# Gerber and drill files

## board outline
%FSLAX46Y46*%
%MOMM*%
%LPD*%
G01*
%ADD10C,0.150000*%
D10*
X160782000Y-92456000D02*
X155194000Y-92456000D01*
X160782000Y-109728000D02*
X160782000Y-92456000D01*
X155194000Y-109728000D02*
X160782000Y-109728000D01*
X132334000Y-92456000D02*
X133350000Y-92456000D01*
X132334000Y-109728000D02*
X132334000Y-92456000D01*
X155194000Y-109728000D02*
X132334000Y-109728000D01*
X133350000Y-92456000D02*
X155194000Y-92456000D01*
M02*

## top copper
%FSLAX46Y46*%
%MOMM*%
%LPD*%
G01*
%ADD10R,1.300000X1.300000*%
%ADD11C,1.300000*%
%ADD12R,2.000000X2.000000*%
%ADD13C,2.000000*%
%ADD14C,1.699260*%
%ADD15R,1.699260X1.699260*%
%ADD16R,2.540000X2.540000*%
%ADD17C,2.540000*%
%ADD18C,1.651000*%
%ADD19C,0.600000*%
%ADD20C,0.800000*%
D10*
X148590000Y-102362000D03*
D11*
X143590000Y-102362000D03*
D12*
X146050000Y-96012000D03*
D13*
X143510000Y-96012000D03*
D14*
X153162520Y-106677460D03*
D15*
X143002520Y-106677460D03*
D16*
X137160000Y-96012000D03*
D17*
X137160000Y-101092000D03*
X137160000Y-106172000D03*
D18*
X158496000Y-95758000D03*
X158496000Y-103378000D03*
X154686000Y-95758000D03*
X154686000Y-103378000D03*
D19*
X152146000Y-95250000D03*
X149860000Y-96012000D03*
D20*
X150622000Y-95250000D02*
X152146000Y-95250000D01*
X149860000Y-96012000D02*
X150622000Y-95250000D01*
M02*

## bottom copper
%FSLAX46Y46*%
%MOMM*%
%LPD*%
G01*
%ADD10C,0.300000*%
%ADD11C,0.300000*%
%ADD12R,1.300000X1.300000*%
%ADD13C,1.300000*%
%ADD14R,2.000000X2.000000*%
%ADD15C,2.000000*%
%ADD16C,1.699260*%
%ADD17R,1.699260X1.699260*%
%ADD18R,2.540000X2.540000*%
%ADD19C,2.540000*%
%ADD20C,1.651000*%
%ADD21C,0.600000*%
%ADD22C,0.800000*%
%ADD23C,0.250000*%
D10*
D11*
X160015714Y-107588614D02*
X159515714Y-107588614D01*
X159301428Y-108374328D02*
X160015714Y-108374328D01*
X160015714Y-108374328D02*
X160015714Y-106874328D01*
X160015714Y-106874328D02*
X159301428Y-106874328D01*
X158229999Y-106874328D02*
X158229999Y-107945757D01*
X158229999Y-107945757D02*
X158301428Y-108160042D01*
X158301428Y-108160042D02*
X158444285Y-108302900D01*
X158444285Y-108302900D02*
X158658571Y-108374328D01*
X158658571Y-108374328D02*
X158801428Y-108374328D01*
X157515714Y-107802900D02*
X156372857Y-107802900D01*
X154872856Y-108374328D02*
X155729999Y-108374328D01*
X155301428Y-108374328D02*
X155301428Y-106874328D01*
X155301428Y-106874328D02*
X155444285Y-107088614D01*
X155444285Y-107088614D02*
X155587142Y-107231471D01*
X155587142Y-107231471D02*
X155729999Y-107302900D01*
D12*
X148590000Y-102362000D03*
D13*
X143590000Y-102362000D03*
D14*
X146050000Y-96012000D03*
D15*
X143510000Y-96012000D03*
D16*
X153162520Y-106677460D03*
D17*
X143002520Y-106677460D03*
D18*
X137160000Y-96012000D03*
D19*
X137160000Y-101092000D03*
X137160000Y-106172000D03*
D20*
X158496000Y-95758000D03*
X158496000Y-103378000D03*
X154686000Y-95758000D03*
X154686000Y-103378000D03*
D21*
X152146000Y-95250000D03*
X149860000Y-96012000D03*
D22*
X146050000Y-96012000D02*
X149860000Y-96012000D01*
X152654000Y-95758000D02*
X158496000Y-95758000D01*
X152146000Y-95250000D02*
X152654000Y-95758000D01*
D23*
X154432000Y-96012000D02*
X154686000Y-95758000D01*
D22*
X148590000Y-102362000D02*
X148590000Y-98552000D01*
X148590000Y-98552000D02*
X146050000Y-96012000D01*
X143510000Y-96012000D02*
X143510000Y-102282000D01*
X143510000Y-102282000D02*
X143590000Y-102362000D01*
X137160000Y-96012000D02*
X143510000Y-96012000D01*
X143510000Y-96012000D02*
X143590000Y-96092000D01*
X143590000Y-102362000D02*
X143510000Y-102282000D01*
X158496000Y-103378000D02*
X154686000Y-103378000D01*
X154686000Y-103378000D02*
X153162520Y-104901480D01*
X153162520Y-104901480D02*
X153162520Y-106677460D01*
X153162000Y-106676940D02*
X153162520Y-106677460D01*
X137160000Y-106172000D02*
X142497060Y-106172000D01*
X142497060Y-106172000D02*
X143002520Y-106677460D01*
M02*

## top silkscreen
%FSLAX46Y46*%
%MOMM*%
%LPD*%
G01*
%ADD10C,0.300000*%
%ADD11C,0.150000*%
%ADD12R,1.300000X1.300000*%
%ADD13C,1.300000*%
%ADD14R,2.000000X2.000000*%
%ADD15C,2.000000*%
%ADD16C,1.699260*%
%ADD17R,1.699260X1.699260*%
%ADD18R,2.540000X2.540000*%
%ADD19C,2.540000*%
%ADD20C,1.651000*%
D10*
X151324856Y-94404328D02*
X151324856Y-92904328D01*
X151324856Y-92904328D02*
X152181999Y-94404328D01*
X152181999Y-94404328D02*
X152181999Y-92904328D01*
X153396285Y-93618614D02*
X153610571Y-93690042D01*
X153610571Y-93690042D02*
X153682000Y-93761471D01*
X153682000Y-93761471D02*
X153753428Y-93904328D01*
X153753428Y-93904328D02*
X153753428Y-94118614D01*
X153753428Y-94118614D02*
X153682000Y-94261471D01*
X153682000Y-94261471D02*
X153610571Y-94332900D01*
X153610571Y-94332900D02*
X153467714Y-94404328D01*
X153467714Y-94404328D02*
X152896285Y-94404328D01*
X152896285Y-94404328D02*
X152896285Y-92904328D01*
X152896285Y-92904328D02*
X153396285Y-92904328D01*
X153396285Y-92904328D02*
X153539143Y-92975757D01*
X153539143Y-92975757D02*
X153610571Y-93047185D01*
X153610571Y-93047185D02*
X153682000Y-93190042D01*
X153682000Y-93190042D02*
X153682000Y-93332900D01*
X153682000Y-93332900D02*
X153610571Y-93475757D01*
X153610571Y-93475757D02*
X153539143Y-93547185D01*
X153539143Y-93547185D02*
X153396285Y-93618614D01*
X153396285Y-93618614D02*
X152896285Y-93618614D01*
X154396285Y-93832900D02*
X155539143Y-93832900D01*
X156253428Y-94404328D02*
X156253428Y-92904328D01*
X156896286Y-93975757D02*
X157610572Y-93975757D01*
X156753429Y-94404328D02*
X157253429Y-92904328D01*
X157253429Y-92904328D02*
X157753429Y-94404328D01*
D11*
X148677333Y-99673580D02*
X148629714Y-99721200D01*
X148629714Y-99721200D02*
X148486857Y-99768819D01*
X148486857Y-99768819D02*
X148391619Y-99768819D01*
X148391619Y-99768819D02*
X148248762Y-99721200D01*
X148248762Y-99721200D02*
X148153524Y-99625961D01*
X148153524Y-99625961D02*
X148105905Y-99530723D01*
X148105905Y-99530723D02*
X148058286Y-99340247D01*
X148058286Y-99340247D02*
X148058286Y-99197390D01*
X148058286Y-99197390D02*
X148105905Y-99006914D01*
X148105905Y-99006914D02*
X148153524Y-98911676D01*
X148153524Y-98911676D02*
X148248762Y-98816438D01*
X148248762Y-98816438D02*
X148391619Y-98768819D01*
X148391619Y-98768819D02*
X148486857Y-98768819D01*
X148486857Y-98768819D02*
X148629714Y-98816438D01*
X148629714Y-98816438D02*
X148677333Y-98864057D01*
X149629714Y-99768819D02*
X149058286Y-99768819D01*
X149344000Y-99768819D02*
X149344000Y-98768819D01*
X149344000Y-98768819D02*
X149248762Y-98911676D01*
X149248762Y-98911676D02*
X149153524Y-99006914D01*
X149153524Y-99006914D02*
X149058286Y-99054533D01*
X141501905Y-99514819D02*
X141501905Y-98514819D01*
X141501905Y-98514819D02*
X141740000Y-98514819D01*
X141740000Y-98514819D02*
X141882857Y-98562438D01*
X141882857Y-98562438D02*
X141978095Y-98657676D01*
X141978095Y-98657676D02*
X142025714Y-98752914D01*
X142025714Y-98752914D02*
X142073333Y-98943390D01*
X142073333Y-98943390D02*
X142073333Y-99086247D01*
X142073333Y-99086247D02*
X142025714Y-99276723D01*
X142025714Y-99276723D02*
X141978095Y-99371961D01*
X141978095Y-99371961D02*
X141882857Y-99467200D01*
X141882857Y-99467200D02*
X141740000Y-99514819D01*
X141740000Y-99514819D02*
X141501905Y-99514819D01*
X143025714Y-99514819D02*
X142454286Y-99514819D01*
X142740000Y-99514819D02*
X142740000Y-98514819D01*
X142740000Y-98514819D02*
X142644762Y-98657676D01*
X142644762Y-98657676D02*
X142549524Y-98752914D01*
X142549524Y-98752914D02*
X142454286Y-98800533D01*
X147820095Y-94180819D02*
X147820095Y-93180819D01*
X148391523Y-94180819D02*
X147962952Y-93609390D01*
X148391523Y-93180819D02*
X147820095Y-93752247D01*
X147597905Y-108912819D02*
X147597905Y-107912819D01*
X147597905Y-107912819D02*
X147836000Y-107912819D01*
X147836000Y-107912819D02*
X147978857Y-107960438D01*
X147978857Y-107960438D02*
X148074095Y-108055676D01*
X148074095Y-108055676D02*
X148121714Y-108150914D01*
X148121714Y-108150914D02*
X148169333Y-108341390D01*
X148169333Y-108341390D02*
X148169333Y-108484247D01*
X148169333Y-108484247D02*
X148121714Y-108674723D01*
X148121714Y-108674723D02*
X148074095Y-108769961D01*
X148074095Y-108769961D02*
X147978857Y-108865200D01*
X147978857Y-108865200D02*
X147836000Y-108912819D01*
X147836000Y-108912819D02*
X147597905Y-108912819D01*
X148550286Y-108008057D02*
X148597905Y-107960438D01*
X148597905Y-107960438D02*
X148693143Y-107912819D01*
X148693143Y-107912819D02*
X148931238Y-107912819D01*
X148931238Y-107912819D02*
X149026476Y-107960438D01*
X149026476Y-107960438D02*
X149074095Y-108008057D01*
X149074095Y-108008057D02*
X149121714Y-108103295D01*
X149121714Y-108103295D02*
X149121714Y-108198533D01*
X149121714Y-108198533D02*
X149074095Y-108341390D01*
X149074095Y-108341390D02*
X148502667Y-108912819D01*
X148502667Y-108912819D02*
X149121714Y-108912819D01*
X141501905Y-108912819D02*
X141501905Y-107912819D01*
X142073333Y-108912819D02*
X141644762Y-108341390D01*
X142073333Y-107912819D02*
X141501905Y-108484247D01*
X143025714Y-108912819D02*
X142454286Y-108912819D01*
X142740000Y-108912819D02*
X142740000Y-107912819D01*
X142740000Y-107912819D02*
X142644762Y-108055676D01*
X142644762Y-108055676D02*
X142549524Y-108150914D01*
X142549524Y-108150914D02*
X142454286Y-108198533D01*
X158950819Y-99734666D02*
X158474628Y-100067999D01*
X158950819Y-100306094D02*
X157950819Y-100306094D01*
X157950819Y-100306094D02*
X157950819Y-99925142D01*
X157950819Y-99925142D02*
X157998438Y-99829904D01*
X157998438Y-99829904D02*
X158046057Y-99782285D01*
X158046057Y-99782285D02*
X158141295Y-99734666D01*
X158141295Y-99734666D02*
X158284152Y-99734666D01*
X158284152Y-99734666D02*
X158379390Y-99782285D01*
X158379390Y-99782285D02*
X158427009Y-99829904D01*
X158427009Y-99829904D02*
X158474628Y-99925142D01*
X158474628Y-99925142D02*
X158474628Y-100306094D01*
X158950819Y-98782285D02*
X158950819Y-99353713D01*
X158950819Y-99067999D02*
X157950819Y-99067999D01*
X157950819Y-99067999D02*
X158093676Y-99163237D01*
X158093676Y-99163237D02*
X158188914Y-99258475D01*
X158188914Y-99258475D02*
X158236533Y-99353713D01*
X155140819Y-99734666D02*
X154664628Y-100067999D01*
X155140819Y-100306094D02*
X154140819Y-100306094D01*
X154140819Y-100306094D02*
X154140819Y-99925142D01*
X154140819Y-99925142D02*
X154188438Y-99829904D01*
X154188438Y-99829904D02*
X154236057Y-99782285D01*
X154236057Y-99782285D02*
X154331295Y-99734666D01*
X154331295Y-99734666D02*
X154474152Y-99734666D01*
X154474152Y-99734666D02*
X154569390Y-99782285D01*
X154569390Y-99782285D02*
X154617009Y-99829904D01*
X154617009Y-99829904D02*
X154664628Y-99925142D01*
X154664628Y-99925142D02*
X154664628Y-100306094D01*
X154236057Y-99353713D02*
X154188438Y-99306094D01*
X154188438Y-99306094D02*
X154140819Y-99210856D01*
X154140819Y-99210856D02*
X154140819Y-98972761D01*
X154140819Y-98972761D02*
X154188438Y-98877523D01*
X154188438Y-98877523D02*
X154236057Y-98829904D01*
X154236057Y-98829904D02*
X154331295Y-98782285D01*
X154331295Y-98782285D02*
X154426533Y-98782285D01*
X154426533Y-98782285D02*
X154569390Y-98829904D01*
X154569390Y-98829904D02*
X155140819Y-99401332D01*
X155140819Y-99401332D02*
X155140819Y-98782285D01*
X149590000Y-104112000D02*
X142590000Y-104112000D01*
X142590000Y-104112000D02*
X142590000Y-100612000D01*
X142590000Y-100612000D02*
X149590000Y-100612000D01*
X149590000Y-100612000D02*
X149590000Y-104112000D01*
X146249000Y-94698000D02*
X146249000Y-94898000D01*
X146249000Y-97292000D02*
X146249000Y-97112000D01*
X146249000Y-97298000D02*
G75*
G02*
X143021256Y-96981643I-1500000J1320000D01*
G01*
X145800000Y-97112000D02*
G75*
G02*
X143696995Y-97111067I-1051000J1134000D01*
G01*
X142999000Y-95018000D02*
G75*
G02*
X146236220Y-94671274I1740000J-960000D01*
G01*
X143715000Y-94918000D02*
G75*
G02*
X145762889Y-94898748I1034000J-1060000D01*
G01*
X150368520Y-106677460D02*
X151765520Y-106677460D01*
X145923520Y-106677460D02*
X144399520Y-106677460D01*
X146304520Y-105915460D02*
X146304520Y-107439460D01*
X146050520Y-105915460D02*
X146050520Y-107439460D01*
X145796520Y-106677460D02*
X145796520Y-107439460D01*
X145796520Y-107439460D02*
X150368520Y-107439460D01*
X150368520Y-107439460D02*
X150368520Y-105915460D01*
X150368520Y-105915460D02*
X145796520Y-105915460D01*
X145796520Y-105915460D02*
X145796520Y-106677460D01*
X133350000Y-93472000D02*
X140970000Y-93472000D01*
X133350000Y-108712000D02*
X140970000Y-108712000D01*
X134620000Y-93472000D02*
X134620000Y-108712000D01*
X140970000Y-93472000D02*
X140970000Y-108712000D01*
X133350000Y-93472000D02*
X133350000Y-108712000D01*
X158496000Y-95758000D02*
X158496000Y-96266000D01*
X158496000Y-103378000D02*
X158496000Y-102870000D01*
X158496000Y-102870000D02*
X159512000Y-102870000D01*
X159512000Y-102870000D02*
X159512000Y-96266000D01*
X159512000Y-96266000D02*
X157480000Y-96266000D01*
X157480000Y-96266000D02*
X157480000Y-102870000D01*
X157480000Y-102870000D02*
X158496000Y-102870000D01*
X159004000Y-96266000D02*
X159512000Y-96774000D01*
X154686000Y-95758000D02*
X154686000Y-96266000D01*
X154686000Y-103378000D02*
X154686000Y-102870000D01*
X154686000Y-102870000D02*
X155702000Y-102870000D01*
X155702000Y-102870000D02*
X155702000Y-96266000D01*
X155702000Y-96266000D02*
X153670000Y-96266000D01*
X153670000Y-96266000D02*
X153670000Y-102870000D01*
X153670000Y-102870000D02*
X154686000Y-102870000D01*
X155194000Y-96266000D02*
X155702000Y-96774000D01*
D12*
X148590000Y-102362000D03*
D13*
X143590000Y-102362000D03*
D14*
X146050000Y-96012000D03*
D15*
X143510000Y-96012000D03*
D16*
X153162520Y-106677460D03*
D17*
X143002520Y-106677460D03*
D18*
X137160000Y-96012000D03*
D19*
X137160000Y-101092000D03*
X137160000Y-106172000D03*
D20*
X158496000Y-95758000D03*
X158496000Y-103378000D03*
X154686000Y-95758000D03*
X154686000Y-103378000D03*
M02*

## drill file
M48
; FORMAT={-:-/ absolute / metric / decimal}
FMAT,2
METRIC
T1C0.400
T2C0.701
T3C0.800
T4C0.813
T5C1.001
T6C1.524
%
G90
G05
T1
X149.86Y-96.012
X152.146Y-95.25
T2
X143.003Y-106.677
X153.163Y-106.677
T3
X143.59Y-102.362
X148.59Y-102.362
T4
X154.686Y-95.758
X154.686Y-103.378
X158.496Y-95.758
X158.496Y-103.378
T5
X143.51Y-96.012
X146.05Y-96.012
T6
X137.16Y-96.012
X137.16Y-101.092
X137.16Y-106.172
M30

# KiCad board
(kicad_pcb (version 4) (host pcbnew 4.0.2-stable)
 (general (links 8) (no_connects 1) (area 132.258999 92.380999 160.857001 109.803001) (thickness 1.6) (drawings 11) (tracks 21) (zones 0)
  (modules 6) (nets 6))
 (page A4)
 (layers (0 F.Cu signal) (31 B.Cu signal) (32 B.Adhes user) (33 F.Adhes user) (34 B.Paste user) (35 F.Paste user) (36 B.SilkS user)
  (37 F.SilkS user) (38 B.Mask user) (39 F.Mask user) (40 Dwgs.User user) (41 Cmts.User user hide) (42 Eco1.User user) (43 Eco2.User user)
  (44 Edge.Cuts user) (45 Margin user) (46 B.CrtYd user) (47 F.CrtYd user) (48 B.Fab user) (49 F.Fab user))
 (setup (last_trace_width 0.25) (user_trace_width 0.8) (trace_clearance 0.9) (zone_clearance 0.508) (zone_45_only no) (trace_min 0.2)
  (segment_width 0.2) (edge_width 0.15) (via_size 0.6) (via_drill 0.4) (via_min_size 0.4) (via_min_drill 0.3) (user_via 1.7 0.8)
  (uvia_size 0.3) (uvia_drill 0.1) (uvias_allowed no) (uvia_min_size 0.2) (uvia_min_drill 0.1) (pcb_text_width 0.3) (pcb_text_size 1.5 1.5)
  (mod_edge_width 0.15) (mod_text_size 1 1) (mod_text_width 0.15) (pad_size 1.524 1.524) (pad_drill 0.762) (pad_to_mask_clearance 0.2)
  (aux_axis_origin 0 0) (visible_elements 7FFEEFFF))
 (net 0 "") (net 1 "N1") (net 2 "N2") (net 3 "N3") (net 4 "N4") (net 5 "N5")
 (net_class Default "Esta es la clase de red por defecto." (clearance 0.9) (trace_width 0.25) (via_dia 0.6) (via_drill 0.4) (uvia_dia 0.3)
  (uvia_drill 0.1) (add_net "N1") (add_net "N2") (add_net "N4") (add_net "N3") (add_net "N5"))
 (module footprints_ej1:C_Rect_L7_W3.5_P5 (layer F.Cu) (at 148.59 102.362 180)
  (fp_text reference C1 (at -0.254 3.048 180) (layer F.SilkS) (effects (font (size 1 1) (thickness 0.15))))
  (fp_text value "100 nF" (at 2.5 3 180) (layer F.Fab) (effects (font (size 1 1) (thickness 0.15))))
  (fp_line (start -1 -1.75) (end 6 -1.75) (layer F.SilkS) (width 0.15))
  (fp_line (start 6 -1.75) (end 6 1.75) (layer F.SilkS) (width 0.15))
  (fp_line (start 6 1.75) (end -1 1.75) (layer F.SilkS) (width 0.15))
  (fp_line (start -1 1.75) (end -1 -1.75) (layer F.SilkS) (width 0.15))
  (pad 1 thru_hole rect (at 0 0 180) (size 1.3 1.3) (drill 0.8) (layers *.Cu *.Mask F.SilkS) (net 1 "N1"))
  (pad 2 thru_hole circle (at 5 0 180) (size 1.3 1.3) (drill 0.8) (layers *.Cu *.Mask F.SilkS) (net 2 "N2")))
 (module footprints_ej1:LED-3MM (layer F.Cu) (at 146.05 96.012 180)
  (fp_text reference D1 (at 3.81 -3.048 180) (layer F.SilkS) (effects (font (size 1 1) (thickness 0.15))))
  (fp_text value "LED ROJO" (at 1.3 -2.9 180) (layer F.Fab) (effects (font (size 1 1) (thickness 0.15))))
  (fp_line (start -0.199 1.314) (end -0.199 1.114) (layer F.SilkS) (width 0.15))
  (fp_line (start -0.199 -1.28) (end -0.199 -1.1) (layer F.SilkS) (width 0.15))
  (fp_arc (start 1.301 0.034) (end -0.199 -1.286) (angle 108.5) (layer F.SilkS) (width 0.15))
  (fp_arc (start 1.301 0.034) (end 0.25 -1.1) (angle 85.7) (layer F.SilkS) (width 0.15))
  (fp_arc (start 1.311 0.034) (end 3.051 0.994) (angle 110) (layer F.SilkS) (width 0.15))
  (fp_arc (start 1.301 0.034) (end 2.335 1.094) (angle 87.5) (layer F.SilkS) (width 0.15))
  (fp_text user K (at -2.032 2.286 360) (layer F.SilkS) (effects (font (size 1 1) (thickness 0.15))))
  (pad 1 thru_hole rect (at 0 0 270) (size 2 2) (drill 1.00076) (layers *.Cu *.Mask F.SilkS) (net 1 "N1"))
  (pad 2 thru_hole circle (at 2.54 0 180) (size 2 2) (drill 1.00076) (layers *.Cu *.Mask F.SilkS) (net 2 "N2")))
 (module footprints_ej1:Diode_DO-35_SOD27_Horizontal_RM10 (layer F.Cu) (at 143.002 106.68)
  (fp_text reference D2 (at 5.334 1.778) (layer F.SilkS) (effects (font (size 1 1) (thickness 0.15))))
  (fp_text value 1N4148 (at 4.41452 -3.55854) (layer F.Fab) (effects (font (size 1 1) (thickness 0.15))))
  (fp_line (start 7.36652 -0.00254) (end 8.76352 -0.00254) (layer F.SilkS) (width 0.15))
  (fp_line (start 2.92152 -0.00254) (end 1.39752 -0.00254) (layer F.SilkS) (width 0.15))
  (fp_line (start 3.30252 -0.76454) (end 3.30252 0.75946) (layer F.SilkS) (width 0.15))
  (fp_line (start 3.04852 -0.76454) (end 3.04852 0.75946) (layer F.SilkS) (width 0.15))
  (fp_line (start 2.79452 -0.00254) (end 2.79452 0.75946) (layer F.SilkS) (width 0.15))
  (fp_line (start 2.79452 0.75946) (end 7.36652 0.75946) (layer F.SilkS) (width 0.15))
  (fp_line (start 7.36652 0.75946) (end 7.36652 -0.76454) (layer F.SilkS) (width 0.15))
  (fp_line (start 7.36652 -0.76454) (end 2.79452 -0.76454) (layer F.SilkS) (width 0.15))
  (fp_line (start 2.79452 -0.76454) (end 2.79452 -0.00254) (layer F.SilkS) (width 0.15))
  (pad 2 thru_hole circle (at 10.16052 -0.00254 180) (size 1.69926 1.69926) (drill 0.70104) (layers *.Cu *.Mask F.SilkS) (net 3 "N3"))
  (pad 1 thru_hole rect (at 0.00052 -0.00254 180) (size 1.69926 1.69926) (drill 0.70104) (layers *.Cu *.Mask F.SilkS) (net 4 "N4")))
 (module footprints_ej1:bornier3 (layer F.Cu) (at 137.16 101.092 270)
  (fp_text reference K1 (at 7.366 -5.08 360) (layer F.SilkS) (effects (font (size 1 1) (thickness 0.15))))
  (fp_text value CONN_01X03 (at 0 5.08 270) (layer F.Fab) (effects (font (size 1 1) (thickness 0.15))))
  (fp_line (start -7.62 3.81) (end -7.62 -3.81) (layer F.SilkS) (width 0.15))
  (fp_line (start 7.62 3.81) (end 7.62 -3.81) (layer F.SilkS) (width 0.15))
  (fp_line (start -7.62 2.54) (end 7.62 2.54) (layer F.SilkS) (width 0.15))
  (fp_line (start -7.62 -3.81) (end 7.62 -3.81) (layer F.SilkS) (width 0.15))
  (fp_line (start -7.62 3.81) (end 7.62 3.81) (layer F.SilkS) (width 0.15))
  (pad 1 thru_hole rect (at -5.08 0 270) (size 2.54 2.54) (drill 1.524) (layers *.Cu *.Mask F.SilkS) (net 2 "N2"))
  (pad 2 thru_hole circle (at 0 0 270) (size 2.54 2.54) (drill 1.524) (layers *.Cu *.Mask F.SilkS) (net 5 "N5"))
  (pad 3 thru_hole circle (at 5.08 0 270) (size 2.54 2.54) (drill 1.524) (layers *.Cu *.Mask F.SilkS) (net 4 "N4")))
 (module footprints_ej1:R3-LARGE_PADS (layer F.Cu) (at 158.496 99.568 270)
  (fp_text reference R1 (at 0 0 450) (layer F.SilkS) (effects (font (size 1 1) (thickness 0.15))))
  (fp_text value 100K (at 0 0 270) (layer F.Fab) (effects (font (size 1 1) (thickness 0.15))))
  (fp_line (start -3.81 0) (end -3.302 0) (layer F.SilkS) (width 0.15))
  (fp_line (start 3.81 0) (end 3.302 0) (layer F.SilkS) (width 0.15))
  (fp_line (start 3.302 0) (end 3.302 -1.016) (layer F.SilkS) (width 0.15))
  (fp_line (start 3.302 -1.016) (end -3.302 -1.016) (layer F.SilkS) (width 0.15))
  (fp_line (start -3.302 -1.016) (end -3.302 1.016) (layer F.SilkS) (width 0.15))
  (fp_line (start -3.302 1.016) (end 3.302 1.016) (layer F.SilkS) (width 0.15))
  (fp_line (start 3.302 1.016) (end 3.302 0) (layer F.SilkS) (width 0.15))
  (fp_line (start -3.302 -0.508) (end -2.794 -1.016) (layer F.SilkS) (width 0.15))
  (pad 1 thru_hole circle (at -3.81 0 270) (size 1.651 1.651) (drill 0.8128) (layers *.Cu *.Mask F.SilkS) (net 1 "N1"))
  (pad 2 thru_hole circle (at 3.81 0 270) (size 1.651 1.651) (drill 0.8128) (layers *.Cu *.Mask F.SilkS) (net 3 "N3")))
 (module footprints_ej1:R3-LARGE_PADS (layer F.Cu) (at 154.686 99.568 270)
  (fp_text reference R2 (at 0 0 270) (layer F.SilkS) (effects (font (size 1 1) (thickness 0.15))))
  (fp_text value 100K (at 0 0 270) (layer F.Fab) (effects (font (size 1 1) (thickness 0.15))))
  (fp_line (start -3.81 0) (end -3.302 0) (layer F.SilkS) (width 0.15))
  (fp_line (start 3.81 0) (end 3.302 0) (layer F.SilkS) (width 0.15))
  (fp_line (start 3.302 0) (end 3.302 -1.016) (layer F.SilkS) (width 0.15))
  (fp_line (start 3.302 -1.016) (end -3.302 -1.016) (layer F.SilkS) (width 0.15))
  (fp_line (start -3.302 -1.016) (end -3.302 1.016) (layer F.SilkS) (width 0.15))
  (fp_line (start -3.302 1.016) (end 3.302 1.016) (layer F.SilkS) (width 0.15))
  (fp_line (start 3.302 1.016) (end 3.302 0) (layer F.SilkS) (width 0.15))
  (fp_line (start -3.302 -0.508) (end -2.794 -1.016) (layer F.SilkS) (width 0.15))
  (pad 1 thru_hole circle (at -3.81 0 270) (size 1.651 1.651) (drill 0.8128) (layers *.Cu *.Mask F.SilkS) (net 1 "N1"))
  (pad 2 thru_hole circle (at 3.81 0 270) (size 1.651 1.651) (drill 0.8128) (layers *.Cu *.Mask F.SilkS) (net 3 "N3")))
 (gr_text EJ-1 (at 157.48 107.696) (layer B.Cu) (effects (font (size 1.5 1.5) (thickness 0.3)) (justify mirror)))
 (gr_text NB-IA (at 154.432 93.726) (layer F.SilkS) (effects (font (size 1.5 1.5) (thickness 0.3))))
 (gr_line (start 160.782 92.456) (end 155.194 92.456) (angle 90) (layer Edge.Cuts) (width 0.15))
 (gr_line (start 160.782 109.728) (end 160.782 92.456) (angle 90) (layer Edge.Cuts) (width 0.15))
 (gr_line (start 155.194 109.728) (end 160.782 109.728) (angle 90) (layer Edge.Cuts) (width 0.15))
 (gr_line (start 132.334 92.456) (end 133.35 92.456) (angle 90) (layer Edge.Cuts) (width 0.15))
 (gr_line (start 132.334 109.728) (end 132.334 92.456) (angle 90) (layer Edge.Cuts) (width 0.15))
 (gr_line (start 155.194 109.728) (end 132.334 109.728) (angle 90) (layer Edge.Cuts) (width 0.15))
 (gr_line (start 133.35 92.456) (end 155.194 92.456) (angle 90) (layer Edge.Cuts) (width 0.15))
 (segment (start 146.05 96.012) (end 149.86 96.012) (width 0.8) (layer B.Cu) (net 1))
 (segment (start 152.654 95.758) (end 158.496 95.758) (width 0.8) (layer B.Cu) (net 1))
 (segment (start 152.146 95.25) (end 152.654 95.758) (width 0.8) (layer B.Cu) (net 1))
 (via (at 152.146 95.25) (size 0.6) (drill 0.4) (layers F.Cu B.Cu) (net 1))
 (segment (start 150.622 95.25) (end 152.146 95.25) (width 0.8) (layer F.Cu) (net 1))
 (segment (start 149.86 96.012) (end 150.622 95.25) (width 0.8) (layer F.Cu) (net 1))
 (via (at 149.86 96.012) (size 0.6) (drill 0.4) (layers F.Cu B.Cu) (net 1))
 (segment (start 154.432 96.012) (end 154.686 95.758) (width 0.25) (layer B.Cu) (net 1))
 (segment (start 148.59 102.362) (end 148.59 98.552) (width 0.8) (layer B.Cu) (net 1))
 (segment (start 148.59 98.552) (end 146.05 96.012) (width 0.8) (layer B.Cu) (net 1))
 (segment (start 143.51 96.012) (end 143.51 102.282) (width 0.8) (layer B.Cu) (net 2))
 (segment (start 143.51 102.282) (end 143.59 102.362) (width 0.8) (layer B.Cu) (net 2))
 (segment (start 137.16 96.012) (end 143.51 96.012) (width 0.8) (layer B.Cu) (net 2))
 (segment (start 143.51 96.012) (end 143.59 96.092) (width 0.8) (layer B.Cu) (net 2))
 (segment (start 143.59 102.362) (end 143.51 102.282) (width 0.8) (layer B.Cu) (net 2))
 (segment (start 158.496 103.378) (end 154.686 103.378) (width 0.8) (layer B.Cu) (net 3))
 (segment (start 154.686 103.378) (end 153.16252 104.90148) (width 0.8) (layer B.Cu) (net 3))
 (segment (start 153.16252 104.90148) (end 153.16252 106.67746) (width 0.8) (layer B.Cu) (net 3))
 (segment (start 153.162 106.67694) (end 153.16252 106.67746) (width 0.8) (layer B.Cu) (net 3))
 (segment (start 137.16 106.172) (end 142.49706 106.172) (width 0.8) (layer B.Cu) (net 4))
 (segment (start 142.49706 106.172) (end 143.00252 106.67746) (width 0.8) (layer B.Cu) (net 4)))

